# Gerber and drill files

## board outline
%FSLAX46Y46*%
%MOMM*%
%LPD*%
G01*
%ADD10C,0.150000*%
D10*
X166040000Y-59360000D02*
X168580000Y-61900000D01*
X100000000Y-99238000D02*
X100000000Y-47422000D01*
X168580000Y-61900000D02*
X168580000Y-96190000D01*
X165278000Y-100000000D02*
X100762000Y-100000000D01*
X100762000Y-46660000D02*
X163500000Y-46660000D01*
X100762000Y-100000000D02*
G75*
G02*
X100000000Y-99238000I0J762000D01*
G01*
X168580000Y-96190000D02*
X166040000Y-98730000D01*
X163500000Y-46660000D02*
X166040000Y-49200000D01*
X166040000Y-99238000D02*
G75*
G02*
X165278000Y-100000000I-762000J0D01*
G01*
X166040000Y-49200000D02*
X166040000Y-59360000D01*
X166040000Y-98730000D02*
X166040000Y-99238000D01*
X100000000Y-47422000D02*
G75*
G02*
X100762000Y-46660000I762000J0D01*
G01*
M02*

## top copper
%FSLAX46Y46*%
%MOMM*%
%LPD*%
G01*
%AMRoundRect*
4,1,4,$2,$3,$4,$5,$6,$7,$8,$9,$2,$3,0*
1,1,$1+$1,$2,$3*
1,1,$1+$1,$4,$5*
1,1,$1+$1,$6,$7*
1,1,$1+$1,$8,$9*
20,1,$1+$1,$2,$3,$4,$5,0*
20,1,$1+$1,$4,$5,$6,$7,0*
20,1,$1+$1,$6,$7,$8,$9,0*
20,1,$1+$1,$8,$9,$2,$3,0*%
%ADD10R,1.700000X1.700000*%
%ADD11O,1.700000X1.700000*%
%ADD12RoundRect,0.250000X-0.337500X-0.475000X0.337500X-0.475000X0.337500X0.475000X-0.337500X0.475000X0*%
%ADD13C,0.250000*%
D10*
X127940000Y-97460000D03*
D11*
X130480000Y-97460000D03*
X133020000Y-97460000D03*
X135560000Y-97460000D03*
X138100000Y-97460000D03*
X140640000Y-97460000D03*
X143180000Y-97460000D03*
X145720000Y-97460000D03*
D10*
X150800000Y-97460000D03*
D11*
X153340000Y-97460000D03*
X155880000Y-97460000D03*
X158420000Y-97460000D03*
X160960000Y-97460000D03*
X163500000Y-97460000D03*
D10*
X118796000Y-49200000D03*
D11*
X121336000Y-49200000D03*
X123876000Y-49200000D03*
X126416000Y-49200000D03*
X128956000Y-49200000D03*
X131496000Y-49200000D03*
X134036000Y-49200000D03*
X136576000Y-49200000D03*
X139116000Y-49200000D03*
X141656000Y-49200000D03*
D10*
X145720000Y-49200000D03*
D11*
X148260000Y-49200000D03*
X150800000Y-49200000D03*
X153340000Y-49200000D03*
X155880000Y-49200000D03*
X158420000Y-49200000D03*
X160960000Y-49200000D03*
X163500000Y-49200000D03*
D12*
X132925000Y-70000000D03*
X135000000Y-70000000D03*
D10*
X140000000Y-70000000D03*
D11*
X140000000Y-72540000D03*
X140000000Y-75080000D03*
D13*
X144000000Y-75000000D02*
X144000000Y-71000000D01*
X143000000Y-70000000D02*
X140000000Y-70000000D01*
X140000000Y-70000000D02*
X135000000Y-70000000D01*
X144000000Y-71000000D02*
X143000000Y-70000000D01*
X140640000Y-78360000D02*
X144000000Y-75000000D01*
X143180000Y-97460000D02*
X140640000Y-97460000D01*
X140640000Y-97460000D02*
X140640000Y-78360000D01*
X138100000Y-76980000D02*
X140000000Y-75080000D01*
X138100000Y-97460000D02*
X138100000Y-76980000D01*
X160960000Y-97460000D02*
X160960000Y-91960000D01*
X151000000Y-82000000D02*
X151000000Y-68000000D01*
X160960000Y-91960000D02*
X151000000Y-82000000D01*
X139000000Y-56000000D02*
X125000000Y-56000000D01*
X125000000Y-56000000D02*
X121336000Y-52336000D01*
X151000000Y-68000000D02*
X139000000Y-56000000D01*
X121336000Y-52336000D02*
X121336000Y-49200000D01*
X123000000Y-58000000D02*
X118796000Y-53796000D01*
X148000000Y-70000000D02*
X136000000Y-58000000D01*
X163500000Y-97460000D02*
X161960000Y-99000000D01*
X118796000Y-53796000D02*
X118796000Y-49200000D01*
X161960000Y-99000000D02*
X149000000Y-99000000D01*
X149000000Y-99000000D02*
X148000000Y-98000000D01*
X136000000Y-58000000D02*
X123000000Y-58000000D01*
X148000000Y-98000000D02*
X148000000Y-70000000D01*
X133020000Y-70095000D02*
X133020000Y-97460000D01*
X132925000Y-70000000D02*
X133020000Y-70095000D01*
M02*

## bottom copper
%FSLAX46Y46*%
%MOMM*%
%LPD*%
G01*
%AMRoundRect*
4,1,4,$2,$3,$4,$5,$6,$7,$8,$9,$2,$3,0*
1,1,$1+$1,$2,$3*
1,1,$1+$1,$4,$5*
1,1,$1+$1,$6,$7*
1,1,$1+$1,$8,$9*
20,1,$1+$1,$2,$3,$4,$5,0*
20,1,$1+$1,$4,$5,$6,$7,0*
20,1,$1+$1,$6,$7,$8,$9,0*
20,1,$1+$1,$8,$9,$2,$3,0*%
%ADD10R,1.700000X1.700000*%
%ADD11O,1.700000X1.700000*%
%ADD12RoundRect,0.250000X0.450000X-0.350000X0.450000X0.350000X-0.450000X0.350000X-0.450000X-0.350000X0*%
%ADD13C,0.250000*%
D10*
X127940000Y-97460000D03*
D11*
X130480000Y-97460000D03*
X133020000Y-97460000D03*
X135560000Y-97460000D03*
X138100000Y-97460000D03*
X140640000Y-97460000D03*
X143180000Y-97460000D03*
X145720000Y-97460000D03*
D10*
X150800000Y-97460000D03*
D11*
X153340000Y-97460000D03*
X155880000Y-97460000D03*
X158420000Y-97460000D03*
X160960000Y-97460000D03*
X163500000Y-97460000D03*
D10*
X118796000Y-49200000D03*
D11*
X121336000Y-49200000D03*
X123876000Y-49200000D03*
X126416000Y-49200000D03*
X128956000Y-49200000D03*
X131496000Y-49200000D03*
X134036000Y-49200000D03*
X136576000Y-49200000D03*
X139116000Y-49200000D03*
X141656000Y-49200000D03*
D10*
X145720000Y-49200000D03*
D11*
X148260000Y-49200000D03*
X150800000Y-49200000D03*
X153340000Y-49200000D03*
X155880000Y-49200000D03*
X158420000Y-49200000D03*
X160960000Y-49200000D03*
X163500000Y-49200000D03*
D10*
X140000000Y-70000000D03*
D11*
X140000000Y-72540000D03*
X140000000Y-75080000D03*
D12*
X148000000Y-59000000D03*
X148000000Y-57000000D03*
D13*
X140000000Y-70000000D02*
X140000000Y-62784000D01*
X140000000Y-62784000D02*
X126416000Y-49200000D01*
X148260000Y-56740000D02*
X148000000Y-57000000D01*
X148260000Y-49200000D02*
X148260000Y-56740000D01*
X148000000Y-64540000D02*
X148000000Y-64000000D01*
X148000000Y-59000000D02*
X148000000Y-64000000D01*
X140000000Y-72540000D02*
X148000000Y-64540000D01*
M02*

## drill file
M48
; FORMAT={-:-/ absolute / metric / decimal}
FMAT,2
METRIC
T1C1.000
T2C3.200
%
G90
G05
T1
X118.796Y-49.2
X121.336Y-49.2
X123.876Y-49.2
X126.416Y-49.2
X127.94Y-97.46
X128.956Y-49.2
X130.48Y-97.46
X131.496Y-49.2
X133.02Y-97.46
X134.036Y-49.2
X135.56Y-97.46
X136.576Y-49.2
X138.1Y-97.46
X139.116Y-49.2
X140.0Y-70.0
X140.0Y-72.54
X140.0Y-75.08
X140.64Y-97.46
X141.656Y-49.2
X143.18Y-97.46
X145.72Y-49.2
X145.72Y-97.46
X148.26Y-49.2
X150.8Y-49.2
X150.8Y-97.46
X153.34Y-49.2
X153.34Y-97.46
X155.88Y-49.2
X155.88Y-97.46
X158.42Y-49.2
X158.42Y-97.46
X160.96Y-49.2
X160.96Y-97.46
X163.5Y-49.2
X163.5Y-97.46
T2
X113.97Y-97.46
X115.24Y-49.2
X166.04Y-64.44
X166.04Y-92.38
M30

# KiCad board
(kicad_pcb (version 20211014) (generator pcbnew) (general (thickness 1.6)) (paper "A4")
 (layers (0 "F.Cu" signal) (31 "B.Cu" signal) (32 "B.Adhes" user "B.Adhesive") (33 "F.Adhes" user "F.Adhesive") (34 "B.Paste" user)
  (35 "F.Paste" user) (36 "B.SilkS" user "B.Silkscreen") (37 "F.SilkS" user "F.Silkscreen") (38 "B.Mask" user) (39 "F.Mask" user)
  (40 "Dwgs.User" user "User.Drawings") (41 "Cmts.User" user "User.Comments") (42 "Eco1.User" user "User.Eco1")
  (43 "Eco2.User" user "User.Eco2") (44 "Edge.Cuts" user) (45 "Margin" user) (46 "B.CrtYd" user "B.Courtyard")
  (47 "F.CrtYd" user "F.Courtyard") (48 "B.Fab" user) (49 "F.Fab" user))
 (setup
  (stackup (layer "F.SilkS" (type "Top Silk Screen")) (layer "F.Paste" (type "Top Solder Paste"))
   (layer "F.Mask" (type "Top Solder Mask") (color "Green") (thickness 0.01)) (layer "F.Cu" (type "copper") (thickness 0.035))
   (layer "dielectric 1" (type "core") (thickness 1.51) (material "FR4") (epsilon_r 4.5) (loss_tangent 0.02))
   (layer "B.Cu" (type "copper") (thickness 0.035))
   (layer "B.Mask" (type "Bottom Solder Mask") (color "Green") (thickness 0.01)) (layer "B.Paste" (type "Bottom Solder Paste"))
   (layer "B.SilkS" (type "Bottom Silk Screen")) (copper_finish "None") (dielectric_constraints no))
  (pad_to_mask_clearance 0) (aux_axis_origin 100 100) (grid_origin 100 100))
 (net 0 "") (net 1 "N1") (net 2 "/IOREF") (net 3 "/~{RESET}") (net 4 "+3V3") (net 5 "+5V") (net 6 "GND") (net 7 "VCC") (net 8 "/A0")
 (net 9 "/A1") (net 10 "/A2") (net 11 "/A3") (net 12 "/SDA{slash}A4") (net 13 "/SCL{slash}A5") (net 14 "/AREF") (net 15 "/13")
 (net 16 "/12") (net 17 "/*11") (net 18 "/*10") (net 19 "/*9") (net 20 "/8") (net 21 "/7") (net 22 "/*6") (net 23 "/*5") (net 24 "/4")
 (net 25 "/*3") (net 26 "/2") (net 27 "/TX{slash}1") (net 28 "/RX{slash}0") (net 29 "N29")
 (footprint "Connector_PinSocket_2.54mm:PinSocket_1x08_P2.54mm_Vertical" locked (layer "F.Cu") (at 127.94 97.46 90)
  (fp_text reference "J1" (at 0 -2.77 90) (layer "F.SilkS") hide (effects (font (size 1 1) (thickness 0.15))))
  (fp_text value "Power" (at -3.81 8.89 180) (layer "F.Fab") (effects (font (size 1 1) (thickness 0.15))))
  (pad "1" thru_hole rect locked (at 0 0 90) (size 1.7 1.7) (drill 1) (layers *.Cu *.Mask) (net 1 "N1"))
  (pad "2" thru_hole oval locked (at 0 2.54 90) (size 1.7 1.7) (drill 1) (layers *.Cu *.Mask) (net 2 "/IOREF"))
  (pad "3" thru_hole oval locked (at 0 5.08 90) (size 1.7 1.7) (drill 1) (layers *.Cu *.Mask) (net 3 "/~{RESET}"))
  (pad "4" thru_hole oval locked (at 0 7.62 90) (size 1.7 1.7) (drill 1) (layers *.Cu *.Mask) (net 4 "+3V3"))
  (pad "5" thru_hole oval locked (at 0 10.16 90) (size 1.7 1.7) (drill 1) (layers *.Cu *.Mask) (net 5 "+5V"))
  (pad "6" thru_hole oval locked (at 0 12.7 90) (size 1.7 1.7) (drill 1) (layers *.Cu *.Mask) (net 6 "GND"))
  (pad "7" thru_hole oval locked (at 0 15.24 90) (size 1.7 1.7) (drill 1) (layers *.Cu *.Mask) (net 6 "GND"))
  (pad "8" thru_hole oval locked (at 0 17.78 90) (size 1.7 1.7) (drill 1) (layers *.Cu *.Mask) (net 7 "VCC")))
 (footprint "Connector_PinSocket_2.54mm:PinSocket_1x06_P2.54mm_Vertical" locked (layer "F.Cu") (at 150.8 97.46 90)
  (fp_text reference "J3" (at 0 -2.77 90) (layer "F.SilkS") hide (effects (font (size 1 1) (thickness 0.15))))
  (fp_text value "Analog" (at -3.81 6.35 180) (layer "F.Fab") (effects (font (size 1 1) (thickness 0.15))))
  (pad "1" thru_hole rect locked (at 0 0 90) (size 1.7 1.7) (drill 1) (layers *.Cu *.Mask) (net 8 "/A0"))
  (pad "2" thru_hole oval locked (at 0 2.54 90) (size 1.7 1.7) (drill 1) (layers *.Cu *.Mask) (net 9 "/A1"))
  (pad "3" thru_hole oval locked (at 0 5.08 90) (size 1.7 1.7) (drill 1) (layers *.Cu *.Mask) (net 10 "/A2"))
  (pad "4" thru_hole oval locked (at 0 7.62 90) (size 1.7 1.7) (drill 1) (layers *.Cu *.Mask) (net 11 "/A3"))
  (pad "5" thru_hole oval locked (at 0 10.16 90) (size 1.7 1.7) (drill 1) (layers *.Cu *.Mask) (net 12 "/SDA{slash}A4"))
  (pad "6" thru_hole oval locked (at 0 12.7 90) (size 1.7 1.7) (drill 1) (layers *.Cu *.Mask) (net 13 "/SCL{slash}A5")))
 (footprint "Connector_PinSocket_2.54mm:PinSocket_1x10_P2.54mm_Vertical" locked (layer "F.Cu") (at 118.796 49.2 90)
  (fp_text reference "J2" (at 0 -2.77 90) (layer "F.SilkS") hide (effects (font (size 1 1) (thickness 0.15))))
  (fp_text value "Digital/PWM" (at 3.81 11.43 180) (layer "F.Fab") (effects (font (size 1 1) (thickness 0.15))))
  (pad "1" thru_hole rect locked (at 0 0 90) (size 1.7 1.7) (drill 1) (layers *.Cu *.Mask) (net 13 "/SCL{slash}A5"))
  (pad "2" thru_hole oval locked (at 0 2.54 90) (size 1.7 1.7) (drill 1) (layers *.Cu *.Mask) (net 12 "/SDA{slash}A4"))
  (pad "3" thru_hole oval locked (at 0 5.08 90) (size 1.7 1.7) (drill 1) (layers *.Cu *.Mask) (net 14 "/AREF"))
  (pad "4" thru_hole oval locked (at 0 7.62 90) (size 1.7 1.7) (drill 1) (layers *.Cu *.Mask) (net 6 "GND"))
  (pad "5" thru_hole oval locked (at 0 10.16 90) (size 1.7 1.7) (drill 1) (layers *.Cu *.Mask) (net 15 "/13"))
  (pad "6" thru_hole oval locked (at 0 12.7 90) (size 1.7 1.7) (drill 1) (layers *.Cu *.Mask) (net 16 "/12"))
  (pad "7" thru_hole oval locked (at 0 15.24 90) (size 1.7 1.7) (drill 1) (layers *.Cu *.Mask) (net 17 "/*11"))
  (pad "8" thru_hole oval locked (at 0 17.78 90) (size 1.7 1.7) (drill 1) (layers *.Cu *.Mask) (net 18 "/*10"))
  (pad "9" thru_hole oval locked (at 0 20.32 90) (size 1.7 1.7) (drill 1) (layers *.Cu *.Mask) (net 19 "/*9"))
  (pad "10" thru_hole oval locked (at 0 22.86 90) (size 1.7 1.7) (drill 1) (layers *.Cu *.Mask) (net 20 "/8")))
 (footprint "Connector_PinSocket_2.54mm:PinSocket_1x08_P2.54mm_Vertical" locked (layer "F.Cu") (at 145.72 49.2 90)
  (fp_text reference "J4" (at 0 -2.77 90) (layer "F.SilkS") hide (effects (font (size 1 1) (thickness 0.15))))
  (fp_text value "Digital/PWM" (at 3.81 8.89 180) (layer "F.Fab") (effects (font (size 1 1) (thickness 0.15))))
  (pad "1" thru_hole rect locked (at 0 0 90) (size 1.7 1.7) (drill 1) (layers *.Cu *.Mask) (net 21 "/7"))
  (pad "2" thru_hole oval locked (at 0 2.54 90) (size 1.7 1.7) (drill 1) (layers *.Cu *.Mask) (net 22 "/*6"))
  (pad "3" thru_hole oval locked (at 0 5.08 90) (size 1.7 1.7) (drill 1) (layers *.Cu *.Mask) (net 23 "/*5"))
  (pad "4" thru_hole oval locked (at 0 7.62 90) (size 1.7 1.7) (drill 1) (layers *.Cu *.Mask) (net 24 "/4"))
  (pad "5" thru_hole oval locked (at 0 10.16 90) (size 1.7 1.7) (drill 1) (layers *.Cu *.Mask) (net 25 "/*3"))
  (pad "6" thru_hole oval locked (at 0 12.7 90) (size 1.7 1.7) (drill 1) (layers *.Cu *.Mask) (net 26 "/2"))
  (pad "7" thru_hole oval locked (at 0 15.24 90) (size 1.7 1.7) (drill 1) (layers *.Cu *.Mask) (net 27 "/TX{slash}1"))
  (pad "8" thru_hole oval locked (at 0 17.78 90) (size 1.7 1.7) (drill 1) (layers *.Cu *.Mask) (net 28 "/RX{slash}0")))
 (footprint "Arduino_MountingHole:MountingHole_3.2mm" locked (layer "F.Cu") (at 115.24 49.2)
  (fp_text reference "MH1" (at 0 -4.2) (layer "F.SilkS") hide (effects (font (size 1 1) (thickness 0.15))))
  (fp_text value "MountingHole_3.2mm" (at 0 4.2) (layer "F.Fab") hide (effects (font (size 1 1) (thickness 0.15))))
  (pad "" np_thru_hole circle locked (at 0 0) (size 3.2 3.2) (drill 3.2) (layers *.Cu *.Mask)))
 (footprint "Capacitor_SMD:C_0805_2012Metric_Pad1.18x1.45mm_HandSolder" (layer "F.Cu") (at 133.9625 70)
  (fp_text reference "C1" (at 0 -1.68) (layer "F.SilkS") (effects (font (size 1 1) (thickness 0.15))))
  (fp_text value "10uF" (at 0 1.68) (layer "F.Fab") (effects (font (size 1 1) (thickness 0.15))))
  (pad "1" smd roundrect (at -1.0375 0) (size 1.175 1.45) (layers "F.Cu" "F.Paste" "F.Mask") (roundrect_rratio 0.2127659574)
   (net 3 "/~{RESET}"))
  (pad "2" smd roundrect (at 1.0375 0) (size 1.175 1.45) (layers "F.Cu" "F.Paste" "F.Mask") (roundrect_rratio 0.2127659574) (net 6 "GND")))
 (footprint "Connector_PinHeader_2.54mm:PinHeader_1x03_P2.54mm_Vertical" (layer "F.Cu") (at 140 70)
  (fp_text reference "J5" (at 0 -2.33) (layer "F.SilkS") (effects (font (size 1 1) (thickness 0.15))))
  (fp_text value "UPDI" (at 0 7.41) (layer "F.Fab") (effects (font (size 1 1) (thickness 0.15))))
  (pad "1" thru_hole rect (at 0 0) (size 1.7 1.7) (drill 1) (layers *.Cu *.Mask) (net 6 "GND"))
  (pad "2" thru_hole oval (at 0 2.54) (size 1.7 1.7) (drill 1) (layers *.Cu *.Mask) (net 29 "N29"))
  (pad "3" thru_hole oval (at 0 5.08) (size 1.7 1.7) (drill 1) (layers *.Cu *.Mask) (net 5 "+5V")))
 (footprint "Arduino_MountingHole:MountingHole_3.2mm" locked (layer "F.Cu") (at 113.97 97.46)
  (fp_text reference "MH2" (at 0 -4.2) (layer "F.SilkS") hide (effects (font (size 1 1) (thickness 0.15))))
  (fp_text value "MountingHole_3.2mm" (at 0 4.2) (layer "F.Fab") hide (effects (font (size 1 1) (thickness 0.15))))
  (pad "" np_thru_hole circle locked (at 0 0) (size 3.2 3.2) (drill 3.2) (layers *.Cu *.Mask)))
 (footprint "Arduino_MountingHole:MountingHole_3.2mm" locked (layer "F.Cu") (at 166.04 64.44)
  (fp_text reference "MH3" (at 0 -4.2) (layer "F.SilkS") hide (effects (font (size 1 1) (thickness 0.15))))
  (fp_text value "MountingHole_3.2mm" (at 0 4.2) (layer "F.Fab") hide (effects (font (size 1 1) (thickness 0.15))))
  (pad "" np_thru_hole circle locked (at 0 0) (size 3.2 3.2) (drill 3.2) (layers *.Cu *.Mask)))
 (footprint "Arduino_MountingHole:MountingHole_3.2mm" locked (layer "F.Cu") (at 166.04 92.38)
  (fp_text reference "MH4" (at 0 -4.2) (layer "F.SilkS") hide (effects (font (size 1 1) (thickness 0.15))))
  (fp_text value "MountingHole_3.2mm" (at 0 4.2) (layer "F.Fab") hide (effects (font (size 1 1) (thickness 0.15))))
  (pad "" np_thru_hole circle locked (at 0 0) (size 3.2 3.2) (drill 3.2) (layers *.Cu *.Mask)))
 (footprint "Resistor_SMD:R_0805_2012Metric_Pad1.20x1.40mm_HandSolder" (layer "B.Cu") (at 148 58 90)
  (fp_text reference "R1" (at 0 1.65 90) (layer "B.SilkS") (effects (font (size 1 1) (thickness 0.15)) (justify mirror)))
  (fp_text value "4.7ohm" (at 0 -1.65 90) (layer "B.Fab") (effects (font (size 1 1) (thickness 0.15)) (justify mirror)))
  (pad "1" smd roundrect (at -1 0 90) (size 1.2 1.4) (layers "B.Cu" "B.Paste" "B.Mask") (roundrect_rratio 0.2083333333) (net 29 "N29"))
  (pad "2" smd roundrect (at 1 0 90) (size 1.2 1.4) (layers "B.Cu" "B.Paste" "B.Mask") (roundrect_rratio 0.2083333333) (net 22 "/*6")))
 (gr_line (start 166.04 59.36) (end 168.58 61.9) (layer "Edge.Cuts") (width 0.15))
 (gr_line (start 100 99.238) (end 100 47.422) (layer "Edge.Cuts") (width 0.15))
 (gr_line (start 168.58 61.9) (end 168.58 96.19) (layer "Edge.Cuts") (width 0.15))
 (gr_line (start 165.278 100) (end 100.762 100) (layer "Edge.Cuts") (width 0.15))
 (gr_line (start 100.762 46.66) (end 163.5 46.66) (layer "Edge.Cuts") (width 0.15))
 (gr_arc (start 100.762 100) (mid 100.223185 99.776815) (end 100 99.238) (layer "Edge.Cuts") (width 0.15))
 (gr_line (start 168.58 96.19) (end 166.04 98.73) (layer "Edge.Cuts") (width 0.15))
 (gr_line (start 163.5 46.66) (end 166.04 49.2) (layer "Edge.Cuts") (width 0.15))
 (gr_arc (start 166.04 99.238) (mid 165.816815 99.776815) (end 165.278 100) (layer "Edge.Cuts") (width 0.15))
 (gr_line (start 166.04 49.2) (end 166.04 59.36) (layer "Edge.Cuts") (width 0.15))
 (gr_line (start 166.04 98.73) (end 166.04 99.238) (layer "Edge.Cuts") (width 0.15))
 (gr_arc (start 100 47.422) (mid 100.223185 46.883185) (end 100.762 46.66) (layer "Edge.Cuts") (width 0.15))
 (segment (start 144 75) (end 144 71) (width 0.25) (layer "F.Cu") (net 6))
 (segment (start 143 70) (end 140 70) (width 0.25) (layer "F.Cu") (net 6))
 (segment (start 140 70) (end 135 70) (width 0.25) (layer "F.Cu") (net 6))
 (segment (start 144 71) (end 143 70) (width 0.25) (layer "F.Cu") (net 6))
 (segment (start 140.64 78.36) (end 144 75) (width 0.25) (layer "F.Cu") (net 6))
 (segment (start 143.18 97.46) (end 140.64 97.46) (width 0.25) (layer "F.Cu") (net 6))
 (segment (start 140.64 97.46) (end 140.64 78.36) (width 0.25) (layer "F.Cu") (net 6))
 (segment (start 140 70) (end 140 62.784) (width 0.25) (layer "B.Cu") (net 6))
 (segment (start 140 62.784) (end 126.416 49.2) (width 0.25) (layer "B.Cu") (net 6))
 (segment (start 138.1 76.98) (end 140 75.08) (width 0.25) (layer "F.Cu") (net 5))
 (segment (start 138.1 97.46) (end 138.1 76.98) (width 0.25) (layer "F.Cu") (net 5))
 (segment (start 160.96 97.46) (end 160.96 91.96) (width 0.25) (layer "F.Cu") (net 12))
 (segment (start 151 82) (end 151 68) (width 0.25) (layer "F.Cu") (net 12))
 (segment (start 160.96 91.96) (end 151 82) (width 0.25) (layer "F.Cu") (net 12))
 (segment (start 139 56) (end 125 56) (width 0.25) (layer "F.Cu") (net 12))
 (segment (start 125 56) (end 121.336 52.336) (width 0.25) (layer "F.Cu") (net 12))
 (segment (start 151 68) (end 139 56) (width 0.25) (layer "F.Cu") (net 12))
 (segment (start 121.336 52.336) (end 121.336 49.2) (width 0.25) (layer "F.Cu") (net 12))
 (segment (start 123 58) (end 118.796 53.796) (width 0.25) (layer "F.Cu") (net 13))
 (segment (start 148 70) (end 136 58) (width 0.25) (layer "F.Cu") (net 13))
 (segment (start 163.5 97.46) (end 161.96 99) (width 0.25) (layer "F.Cu") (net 13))
 (segment (start 118.796 53.796) (end 118.796 49.2) (width 0.25) (layer "F.Cu") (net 13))
 (segment (start 161.96 99) (end 149 99) (width 0.25) (layer "F.Cu") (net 13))
 (segment (start 149 99) (end 148 98) (width 0.25) (layer "F.Cu") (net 13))
 (segment (start 136 58) (end 123 58) (width 0.25) (layer "F.Cu") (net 13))
 (segment (start 148 98) (end 148 70) (width 0.25) (layer "F.Cu") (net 13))
 (segment (start 148.26 56.74) (end 148 57) (width 0.25) (layer "B.Cu") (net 22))
 (segment (start 148.26 49.2) (end 148.26 56.74) (width 0.25) (layer "B.Cu") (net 22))
 (segment (start 133.02 70.095) (end 133.02 97.46) (width 0.25) (layer "F.Cu") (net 3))
 (segment (start 132.925 70) (end 133.02 70.095) (width 0.25) (layer "F.Cu") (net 3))
 (segment (start 148 64.54) (end 148 64) (width 0.25) (layer "B.Cu") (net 29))
 (segment (start 148 59) (end 148 64) (width 0.25) (layer "B.Cu") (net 29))
 (segment (start 140 72.54) (end 148 64.54) (width 0.25) (layer "B.Cu") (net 29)))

